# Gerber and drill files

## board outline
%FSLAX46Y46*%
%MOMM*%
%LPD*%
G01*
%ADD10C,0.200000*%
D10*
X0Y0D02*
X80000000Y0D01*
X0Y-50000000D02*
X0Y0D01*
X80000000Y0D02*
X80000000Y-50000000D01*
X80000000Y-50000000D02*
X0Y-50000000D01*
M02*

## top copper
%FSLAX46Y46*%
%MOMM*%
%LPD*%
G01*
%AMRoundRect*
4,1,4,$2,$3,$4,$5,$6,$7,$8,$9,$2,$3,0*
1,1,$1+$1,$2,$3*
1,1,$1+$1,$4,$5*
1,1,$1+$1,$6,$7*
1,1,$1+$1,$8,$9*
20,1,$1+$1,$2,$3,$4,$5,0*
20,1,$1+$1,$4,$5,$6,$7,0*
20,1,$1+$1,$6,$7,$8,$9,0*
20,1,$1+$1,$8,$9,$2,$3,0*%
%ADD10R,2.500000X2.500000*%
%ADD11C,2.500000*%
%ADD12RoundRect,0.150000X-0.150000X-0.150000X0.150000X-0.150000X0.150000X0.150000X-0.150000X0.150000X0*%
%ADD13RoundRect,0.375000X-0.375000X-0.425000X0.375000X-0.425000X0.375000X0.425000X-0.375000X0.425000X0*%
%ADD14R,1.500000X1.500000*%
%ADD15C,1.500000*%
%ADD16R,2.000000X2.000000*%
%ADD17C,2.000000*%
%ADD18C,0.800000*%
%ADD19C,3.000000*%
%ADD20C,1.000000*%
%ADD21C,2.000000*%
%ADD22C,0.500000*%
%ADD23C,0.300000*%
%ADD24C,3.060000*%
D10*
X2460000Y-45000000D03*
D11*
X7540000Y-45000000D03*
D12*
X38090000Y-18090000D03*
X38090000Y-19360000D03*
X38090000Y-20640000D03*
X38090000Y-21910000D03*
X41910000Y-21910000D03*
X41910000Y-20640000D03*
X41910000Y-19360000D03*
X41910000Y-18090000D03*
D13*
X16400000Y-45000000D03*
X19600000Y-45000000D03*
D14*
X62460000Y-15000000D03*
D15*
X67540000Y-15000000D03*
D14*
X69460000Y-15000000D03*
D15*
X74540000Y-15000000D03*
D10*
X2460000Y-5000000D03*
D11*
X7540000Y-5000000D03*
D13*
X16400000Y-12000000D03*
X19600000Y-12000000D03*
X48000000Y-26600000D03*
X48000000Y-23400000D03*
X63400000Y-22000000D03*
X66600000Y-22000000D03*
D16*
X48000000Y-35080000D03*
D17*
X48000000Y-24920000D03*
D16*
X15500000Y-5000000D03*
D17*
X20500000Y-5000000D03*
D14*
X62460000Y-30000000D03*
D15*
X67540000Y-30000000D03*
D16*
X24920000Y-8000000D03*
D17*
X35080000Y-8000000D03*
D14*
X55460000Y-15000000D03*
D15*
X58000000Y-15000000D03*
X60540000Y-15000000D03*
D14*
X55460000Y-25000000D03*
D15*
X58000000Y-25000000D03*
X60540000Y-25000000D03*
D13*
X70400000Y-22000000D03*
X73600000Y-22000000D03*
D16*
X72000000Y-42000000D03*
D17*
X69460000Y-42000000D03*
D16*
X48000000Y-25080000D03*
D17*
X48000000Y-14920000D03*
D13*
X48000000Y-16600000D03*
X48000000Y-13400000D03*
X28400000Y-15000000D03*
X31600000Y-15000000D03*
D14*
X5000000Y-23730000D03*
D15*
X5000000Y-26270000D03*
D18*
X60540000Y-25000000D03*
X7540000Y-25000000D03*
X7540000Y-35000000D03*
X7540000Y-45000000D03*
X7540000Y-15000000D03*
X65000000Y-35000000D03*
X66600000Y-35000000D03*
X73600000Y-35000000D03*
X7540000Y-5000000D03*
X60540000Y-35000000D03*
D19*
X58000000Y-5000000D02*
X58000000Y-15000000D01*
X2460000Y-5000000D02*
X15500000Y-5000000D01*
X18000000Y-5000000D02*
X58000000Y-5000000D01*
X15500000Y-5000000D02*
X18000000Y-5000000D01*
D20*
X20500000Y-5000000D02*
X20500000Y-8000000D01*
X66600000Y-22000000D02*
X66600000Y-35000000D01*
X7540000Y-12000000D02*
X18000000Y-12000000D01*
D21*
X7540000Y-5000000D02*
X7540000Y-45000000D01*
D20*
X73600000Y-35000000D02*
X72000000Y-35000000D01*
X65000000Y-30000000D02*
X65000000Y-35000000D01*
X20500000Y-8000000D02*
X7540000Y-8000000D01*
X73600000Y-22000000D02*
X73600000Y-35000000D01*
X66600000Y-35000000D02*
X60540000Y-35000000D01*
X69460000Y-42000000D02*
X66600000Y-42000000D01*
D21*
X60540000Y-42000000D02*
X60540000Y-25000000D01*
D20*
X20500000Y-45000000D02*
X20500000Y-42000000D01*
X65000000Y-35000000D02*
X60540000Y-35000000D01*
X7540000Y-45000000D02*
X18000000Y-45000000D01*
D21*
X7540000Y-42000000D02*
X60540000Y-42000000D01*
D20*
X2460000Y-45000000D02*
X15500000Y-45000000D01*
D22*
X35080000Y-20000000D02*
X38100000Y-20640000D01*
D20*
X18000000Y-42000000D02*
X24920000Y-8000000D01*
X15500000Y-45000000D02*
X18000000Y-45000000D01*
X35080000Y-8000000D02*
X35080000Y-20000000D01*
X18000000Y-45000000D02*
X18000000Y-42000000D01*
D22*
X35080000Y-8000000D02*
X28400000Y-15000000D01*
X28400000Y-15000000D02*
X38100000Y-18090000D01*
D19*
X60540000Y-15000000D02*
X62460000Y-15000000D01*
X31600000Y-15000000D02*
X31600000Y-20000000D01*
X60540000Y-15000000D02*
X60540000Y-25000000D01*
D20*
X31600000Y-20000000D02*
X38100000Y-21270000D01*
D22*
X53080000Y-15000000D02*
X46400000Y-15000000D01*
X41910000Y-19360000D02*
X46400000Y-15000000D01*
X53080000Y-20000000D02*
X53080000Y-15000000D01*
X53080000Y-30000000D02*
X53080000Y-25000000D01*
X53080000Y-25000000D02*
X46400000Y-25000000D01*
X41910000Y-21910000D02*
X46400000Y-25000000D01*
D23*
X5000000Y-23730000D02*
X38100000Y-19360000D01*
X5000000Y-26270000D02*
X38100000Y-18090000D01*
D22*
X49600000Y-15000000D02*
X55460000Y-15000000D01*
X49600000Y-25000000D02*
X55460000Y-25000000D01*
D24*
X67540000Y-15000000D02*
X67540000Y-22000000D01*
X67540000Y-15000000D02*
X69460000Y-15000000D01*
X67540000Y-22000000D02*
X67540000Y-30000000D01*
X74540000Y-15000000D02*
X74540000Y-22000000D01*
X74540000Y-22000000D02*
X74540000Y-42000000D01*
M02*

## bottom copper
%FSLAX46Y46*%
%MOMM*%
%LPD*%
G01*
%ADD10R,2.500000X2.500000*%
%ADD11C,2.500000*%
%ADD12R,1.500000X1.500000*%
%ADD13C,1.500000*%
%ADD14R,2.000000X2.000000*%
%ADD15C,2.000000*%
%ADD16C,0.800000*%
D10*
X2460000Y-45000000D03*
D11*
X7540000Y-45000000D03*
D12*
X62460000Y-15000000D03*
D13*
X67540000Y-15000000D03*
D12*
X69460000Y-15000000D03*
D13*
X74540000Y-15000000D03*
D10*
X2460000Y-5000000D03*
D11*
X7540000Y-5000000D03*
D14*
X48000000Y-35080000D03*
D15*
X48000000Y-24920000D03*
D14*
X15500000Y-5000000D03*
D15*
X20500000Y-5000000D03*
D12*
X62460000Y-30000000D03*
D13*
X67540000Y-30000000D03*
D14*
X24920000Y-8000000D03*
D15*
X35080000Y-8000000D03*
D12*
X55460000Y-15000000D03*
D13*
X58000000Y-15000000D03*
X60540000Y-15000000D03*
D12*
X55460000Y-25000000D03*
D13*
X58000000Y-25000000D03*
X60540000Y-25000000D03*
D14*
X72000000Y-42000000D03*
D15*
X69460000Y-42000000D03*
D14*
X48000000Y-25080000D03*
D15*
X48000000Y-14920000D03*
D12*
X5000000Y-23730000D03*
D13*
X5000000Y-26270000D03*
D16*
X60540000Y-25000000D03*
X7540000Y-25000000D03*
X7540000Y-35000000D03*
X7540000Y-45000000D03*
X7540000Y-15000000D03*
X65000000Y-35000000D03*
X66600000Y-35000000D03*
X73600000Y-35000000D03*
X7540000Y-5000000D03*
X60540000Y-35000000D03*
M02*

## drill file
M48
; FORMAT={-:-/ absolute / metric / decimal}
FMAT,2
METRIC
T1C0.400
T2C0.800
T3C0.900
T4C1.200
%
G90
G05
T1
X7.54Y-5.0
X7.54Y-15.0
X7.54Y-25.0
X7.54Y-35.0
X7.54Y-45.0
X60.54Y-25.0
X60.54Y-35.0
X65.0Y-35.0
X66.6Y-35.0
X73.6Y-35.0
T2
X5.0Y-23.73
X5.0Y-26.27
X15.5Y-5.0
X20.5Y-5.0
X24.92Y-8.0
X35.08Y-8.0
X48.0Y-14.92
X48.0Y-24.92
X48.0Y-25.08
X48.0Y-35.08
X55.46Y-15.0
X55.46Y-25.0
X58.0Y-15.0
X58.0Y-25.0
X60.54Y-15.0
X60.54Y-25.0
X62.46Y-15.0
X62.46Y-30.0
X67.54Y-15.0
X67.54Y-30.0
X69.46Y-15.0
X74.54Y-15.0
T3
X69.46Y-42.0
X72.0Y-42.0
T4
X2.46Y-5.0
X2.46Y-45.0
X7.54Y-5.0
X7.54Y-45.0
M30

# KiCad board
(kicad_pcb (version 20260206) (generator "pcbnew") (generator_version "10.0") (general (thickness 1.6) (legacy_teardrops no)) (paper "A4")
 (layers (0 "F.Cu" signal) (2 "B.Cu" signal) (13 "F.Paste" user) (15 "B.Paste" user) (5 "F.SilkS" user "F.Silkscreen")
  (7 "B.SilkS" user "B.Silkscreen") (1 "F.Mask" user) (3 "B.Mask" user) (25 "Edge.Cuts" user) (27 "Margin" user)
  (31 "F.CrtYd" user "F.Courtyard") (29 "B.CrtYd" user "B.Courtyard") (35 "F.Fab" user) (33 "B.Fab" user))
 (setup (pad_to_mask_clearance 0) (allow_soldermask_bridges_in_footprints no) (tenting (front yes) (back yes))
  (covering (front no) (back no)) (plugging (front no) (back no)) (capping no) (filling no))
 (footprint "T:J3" (layer "F.Cu") (at 5 45)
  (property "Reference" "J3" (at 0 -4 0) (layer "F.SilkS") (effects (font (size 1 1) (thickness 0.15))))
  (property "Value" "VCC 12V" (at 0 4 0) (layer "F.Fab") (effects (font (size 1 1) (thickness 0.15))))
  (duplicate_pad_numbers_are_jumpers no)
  (pad "1" thru_hole rect (at -2.54 0) (size 2.5 2.5) (drill 1.2) (layers "*.Cu" "*.Mask") (remove_unused_layers no) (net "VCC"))
  (pad "2" thru_hole circle (at 2.54 0) (size 2.5 2.5) (drill 1.2) (layers "*.Cu" "*.Mask") (remove_unused_layers no) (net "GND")))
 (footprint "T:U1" (layer "F.Cu") (at 40 20)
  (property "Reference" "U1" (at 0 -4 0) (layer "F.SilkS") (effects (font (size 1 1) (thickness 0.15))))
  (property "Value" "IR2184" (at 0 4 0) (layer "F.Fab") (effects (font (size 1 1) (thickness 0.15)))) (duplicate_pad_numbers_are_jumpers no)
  (pad "1" smd roundrect (at -1.91 -1.91) (size 0.6 0.6) (layers "F.Cu" "F.Mask" "F.Paste") (roundrect_rratio 0.25) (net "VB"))
  (pad "2" smd roundrect (at -1.91 -0.64) (size 0.6 0.6) (layers "F.Cu" "F.Mask" "F.Paste") (roundrect_rratio 0.25) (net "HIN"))
  (pad "3" smd roundrect (at -1.91 0.64) (size 0.6 0.6) (layers "F.Cu" "F.Mask" "F.Paste") (roundrect_rratio 0.25) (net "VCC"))
  (pad "4" smd roundrect (at -1.91 1.91) (size 0.6 0.6) (layers "F.Cu" "F.Mask" "F.Paste") (roundrect_rratio 0.25) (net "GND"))
  (pad "5" smd roundrect (at 1.91 1.91) (size 0.6 0.6) (layers "F.Cu" "F.Mask" "F.Paste") (roundrect_rratio 0.25) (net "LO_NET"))
  (pad "6" smd roundrect (at 1.91 0.64) (size 0.6 0.6) (layers "F.Cu" "F.Mask" "F.Paste") (roundrect_rratio 0.25) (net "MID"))
  (pad "7" smd roundrect (at 1.91 -0.64) (size 0.6 0.6) (layers "F.Cu" "F.Mask" "F.Paste") (roundrect_rratio 0.25) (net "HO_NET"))
  (pad "8" smd roundrect (at 1.91 -1.91) (size 0.6 0.6) (layers "F.Cu" "F.Mask" "F.Paste") (roundrect_rratio 0.25) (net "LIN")))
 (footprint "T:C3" (layer "F.Cu") (at 18 45)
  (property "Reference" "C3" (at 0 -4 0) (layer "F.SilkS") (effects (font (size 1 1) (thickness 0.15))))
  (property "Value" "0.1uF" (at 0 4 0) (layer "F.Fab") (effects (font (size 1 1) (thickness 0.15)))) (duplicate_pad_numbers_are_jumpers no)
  (pad "1" smd roundrect (at -1.6 0) (size 1.5 1.6) (layers "F.Cu" "F.Mask" "F.Paste") (roundrect_rratio 0.25) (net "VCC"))
  (pad "2" smd roundrect (at 1.6 0) (size 1.5 1.6) (layers "F.Cu" "F.Mask" "F.Paste") (roundrect_rratio 0.25) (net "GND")))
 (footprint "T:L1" (layer "F.Cu") (at 65 15)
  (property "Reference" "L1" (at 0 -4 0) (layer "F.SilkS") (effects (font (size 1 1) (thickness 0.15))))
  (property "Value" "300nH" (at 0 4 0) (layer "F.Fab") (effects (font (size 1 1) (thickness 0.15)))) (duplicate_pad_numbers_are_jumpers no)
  (pad "1" thru_hole rect (at -2.54 0) (size 1.5 1.5) (drill 0.8) (layers "*.Cu" "*.Mask") (remove_unused_layers no) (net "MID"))
  (pad "2" thru_hole circle (at 2.54 0) (size 1.5 1.5) (drill 0.8) (layers "*.Cu" "*.Mask") (remove_unused_layers no) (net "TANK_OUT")))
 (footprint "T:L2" (layer "F.Cu") (at 72 15)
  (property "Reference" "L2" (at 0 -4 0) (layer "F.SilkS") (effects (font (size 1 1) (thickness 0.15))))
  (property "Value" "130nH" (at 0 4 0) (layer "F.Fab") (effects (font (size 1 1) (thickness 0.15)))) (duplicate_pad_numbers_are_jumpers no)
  (pad "1" thru_hole rect (at -2.54 0) (size 1.5 1.5) (drill 0.8) (layers "*.Cu" "*.Mask") (remove_unused_layers no) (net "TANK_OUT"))
  (pad "2" thru_hole circle (at 2.54 0) (size 1.5 1.5) (drill 0.8) (layers "*.Cu" "*.Mask") (remove_unused_layers no) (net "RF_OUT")))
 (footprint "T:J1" (layer "F.Cu") (at 5 5)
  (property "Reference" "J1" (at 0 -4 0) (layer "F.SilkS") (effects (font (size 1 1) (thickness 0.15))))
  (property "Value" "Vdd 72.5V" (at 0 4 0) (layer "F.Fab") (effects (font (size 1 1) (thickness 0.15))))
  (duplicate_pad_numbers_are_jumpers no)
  (pad "1" thru_hole rect (at -2.54 0) (size 2.5 2.5) (drill 1.2) (layers "*.Cu" "*.Mask") (remove_unused_layers no) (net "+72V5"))
  (pad "2" thru_hole circle (at 2.54 0) (size 2.5 2.5) (drill 1.2) (layers "*.Cu" "*.Mask") (remove_unused_layers no) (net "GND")))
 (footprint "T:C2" (layer "F.Cu") (at 18 12)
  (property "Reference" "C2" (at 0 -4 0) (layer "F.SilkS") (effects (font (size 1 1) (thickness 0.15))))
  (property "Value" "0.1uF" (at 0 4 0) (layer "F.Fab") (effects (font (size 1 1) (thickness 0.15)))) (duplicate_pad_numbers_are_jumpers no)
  (pad "1" smd roundrect (at -1.6 0) (size 1.5 1.6) (layers "F.Cu" "F.Mask" "F.Paste") (roundrect_rratio 0.25) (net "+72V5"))
  (pad "2" smd roundrect (at 1.6 0) (size 1.5 1.6) (layers "F.Cu" "F.Mask" "F.Paste") (roundrect_rratio 0.25) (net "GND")))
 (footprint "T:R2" (layer "F.Cu") (at 48 25 90)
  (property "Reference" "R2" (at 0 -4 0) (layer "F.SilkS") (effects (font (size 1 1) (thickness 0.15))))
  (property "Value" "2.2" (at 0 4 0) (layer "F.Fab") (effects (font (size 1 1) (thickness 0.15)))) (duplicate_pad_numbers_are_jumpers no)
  (pad "1" smd roundrect (at -1.6 0) (size 1.5 1.6) (layers "F.Cu" "F.Mask" "F.Paste") (roundrect_rratio 0.25) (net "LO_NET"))
  (pad "2" smd roundrect (at 1.6 0) (size 1.5 1.6) (layers "F.Cu" "F.Mask" "F.Paste") (roundrect_rratio 0.25) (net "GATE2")))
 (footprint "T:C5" (layer "F.Cu") (at 65 22)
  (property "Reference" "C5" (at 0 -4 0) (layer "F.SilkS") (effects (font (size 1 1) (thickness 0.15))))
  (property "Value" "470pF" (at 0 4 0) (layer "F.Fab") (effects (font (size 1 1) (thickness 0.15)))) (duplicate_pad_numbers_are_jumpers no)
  (pad "1" smd roundrect (at -1.6 0) (size 1.5 1.6) (layers "F.Cu" "F.Mask" "F.Paste") (roundrect_rratio 0.25) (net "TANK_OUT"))
  (pad "2" smd roundrect (at 1.6 0) (size 1.5 1.6) (layers "F.Cu" "F.Mask" "F.Paste") (roundrect_rratio 0.25) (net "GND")))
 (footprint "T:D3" (layer "F.Cu") (at 48 30 90)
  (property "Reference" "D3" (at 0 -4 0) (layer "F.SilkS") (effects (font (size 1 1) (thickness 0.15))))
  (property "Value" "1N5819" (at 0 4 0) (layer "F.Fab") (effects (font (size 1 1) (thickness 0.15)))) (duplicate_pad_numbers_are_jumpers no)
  (pad "1" thru_hole rect (at -5.08 0) (size 2 2) (drill 0.8) (layers "*.Cu" "*.Mask") (remove_unused_layers no) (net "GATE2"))
  (pad "2" thru_hole circle (at 5.08 0) (size 2 2) (drill 0.8) (layers "*.Cu" "*.Mask") (remove_unused_layers no) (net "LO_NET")))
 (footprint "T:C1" (layer "F.Cu") (at 18 5)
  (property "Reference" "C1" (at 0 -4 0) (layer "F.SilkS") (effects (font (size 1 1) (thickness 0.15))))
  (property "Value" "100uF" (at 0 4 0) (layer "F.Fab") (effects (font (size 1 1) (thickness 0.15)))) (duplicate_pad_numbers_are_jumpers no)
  (pad "1" thru_hole rect (at -2.5 0) (size 2 2) (drill 0.8) (layers "*.Cu" "*.Mask") (remove_unused_layers no) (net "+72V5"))
  (pad "2" thru_hole circle (at 2.5 0) (size 2 2) (drill 0.8) (layers "*.Cu" "*.Mask") (remove_unused_layers no) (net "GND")))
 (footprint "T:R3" (layer "F.Cu") (at 65 30)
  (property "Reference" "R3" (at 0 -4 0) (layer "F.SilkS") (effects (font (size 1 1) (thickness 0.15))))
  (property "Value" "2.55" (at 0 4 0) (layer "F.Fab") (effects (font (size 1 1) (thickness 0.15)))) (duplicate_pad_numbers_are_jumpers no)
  (pad "1" thru_hole rect (at -2.54 0) (size 1.5 1.5) (drill 0.8) (layers "*.Cu" "*.Mask") (remove_unused_layers no) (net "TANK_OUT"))
  (pad "2" thru_hole circle (at 2.54 0) (size 1.5 1.5) (drill 0.8) (layers "*.Cu" "*.Mask") (remove_unused_layers no) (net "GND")))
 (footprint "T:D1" (layer "F.Cu") (at 30 8)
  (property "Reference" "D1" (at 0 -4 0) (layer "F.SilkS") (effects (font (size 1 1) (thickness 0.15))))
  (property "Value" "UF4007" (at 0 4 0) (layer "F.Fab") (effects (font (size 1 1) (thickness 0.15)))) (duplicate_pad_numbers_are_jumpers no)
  (pad "1" thru_hole rect (at -5.08 0) (size 2 2) (drill 0.8) (layers "*.Cu" "*.Mask") (remove_unused_layers no) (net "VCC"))
  (pad "2" thru_hole circle (at 5.08 0) (size 2 2) (drill 0.8) (layers "*.Cu" "*.Mask") (remove_unused_layers no) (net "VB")))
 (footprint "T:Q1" (layer "F.Cu") (at 58 15)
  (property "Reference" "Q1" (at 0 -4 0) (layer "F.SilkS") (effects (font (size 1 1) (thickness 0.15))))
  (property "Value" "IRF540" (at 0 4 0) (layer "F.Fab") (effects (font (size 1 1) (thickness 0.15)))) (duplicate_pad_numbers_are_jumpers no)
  (pad "1" thru_hole rect (at -2.54 0) (size 1.5 1.5) (drill 0.8) (layers "*.Cu" "*.Mask") (remove_unused_layers no) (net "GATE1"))
  (pad "2" thru_hole circle (at 0 0) (size 1.5 1.5) (drill 0.8) (layers "*.Cu" "*.Mask") (remove_unused_layers no) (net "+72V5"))
  (pad "3" thru_hole circle (at 2.54 0) (size 1.5 1.5) (drill 0.8) (layers "*.Cu" "*.Mask") (remove_unused_layers no) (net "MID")))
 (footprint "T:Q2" (layer "F.Cu") (at 58 25)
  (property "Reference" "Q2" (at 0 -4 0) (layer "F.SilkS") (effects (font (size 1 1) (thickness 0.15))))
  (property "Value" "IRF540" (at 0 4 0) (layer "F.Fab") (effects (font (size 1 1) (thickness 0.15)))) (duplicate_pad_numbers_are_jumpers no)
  (pad "1" thru_hole rect (at -2.54 0) (size 1.5 1.5) (drill 0.8) (layers "*.Cu" "*.Mask") (remove_unused_layers no) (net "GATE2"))
  (pad "2" thru_hole circle (at 0 0) (size 1.5 1.5) (drill 0.8) (layers "*.Cu" "*.Mask") (remove_unused_layers no) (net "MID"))
  (pad "3" thru_hole circle (at 2.54 0) (size 1.5 1.5) (drill 0.8) (layers "*.Cu" "*.Mask") (remove_unused_layers no) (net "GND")))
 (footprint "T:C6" (layer "F.Cu") (at 72 22)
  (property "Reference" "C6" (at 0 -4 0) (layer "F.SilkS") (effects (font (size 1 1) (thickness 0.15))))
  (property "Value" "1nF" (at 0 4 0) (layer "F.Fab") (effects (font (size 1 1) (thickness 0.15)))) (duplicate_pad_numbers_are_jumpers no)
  (pad "1" smd roundrect (at -1.6 0) (size 1.5 1.6) (layers "F.Cu" "F.Mask" "F.Paste") (roundrect_rratio 0.25) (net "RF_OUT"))
  (pad "2" smd roundrect (at 1.6 0) (size 1.5 1.6) (layers "F.Cu" "F.Mask" "F.Paste") (roundrect_rratio 0.25) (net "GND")))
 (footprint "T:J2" (layer "F.Cu") (at 72 42)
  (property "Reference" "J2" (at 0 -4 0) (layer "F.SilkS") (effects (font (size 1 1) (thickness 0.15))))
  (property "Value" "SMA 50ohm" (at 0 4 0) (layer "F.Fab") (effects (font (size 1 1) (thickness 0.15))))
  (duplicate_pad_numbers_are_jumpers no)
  (pad "1" thru_hole rect (at 0 0) (size 2 2) (drill 0.9) (layers "*.Cu" "*.Mask") (remove_unused_layers no) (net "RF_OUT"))
  (pad "2" thru_hole circle (at -2.54 0) (size 2 2) (drill 0.9) (layers "*.Cu" "*.Mask") (remove_unused_layers no) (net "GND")))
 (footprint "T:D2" (layer "F.Cu") (at 48 20 90)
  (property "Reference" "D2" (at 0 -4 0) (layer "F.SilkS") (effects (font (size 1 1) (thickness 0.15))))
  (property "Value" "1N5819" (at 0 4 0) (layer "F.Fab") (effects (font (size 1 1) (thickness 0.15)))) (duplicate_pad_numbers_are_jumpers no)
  (pad "1" thru_hole rect (at -5.08 0) (size 2 2) (drill 0.8) (layers "*.Cu" "*.Mask") (remove_unused_layers no) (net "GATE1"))
  (pad "2" thru_hole circle (at 5.08 0) (size 2 2) (drill 0.8) (layers "*.Cu" "*.Mask") (remove_unused_layers no) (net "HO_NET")))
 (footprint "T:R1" (layer "F.Cu") (at 48 15 90)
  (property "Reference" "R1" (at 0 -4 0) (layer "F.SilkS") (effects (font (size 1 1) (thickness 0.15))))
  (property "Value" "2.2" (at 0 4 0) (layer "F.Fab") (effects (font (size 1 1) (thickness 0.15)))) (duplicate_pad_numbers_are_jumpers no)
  (pad "1" smd roundrect (at -1.6 0) (size 1.5 1.6) (layers "F.Cu" "F.Mask" "F.Paste") (roundrect_rratio 0.25) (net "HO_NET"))
  (pad "2" smd roundrect (at 1.6 0) (size 1.5 1.6) (layers "F.Cu" "F.Mask" "F.Paste") (roundrect_rratio 0.25) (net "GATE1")))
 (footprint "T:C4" (layer "F.Cu") (at 30 15)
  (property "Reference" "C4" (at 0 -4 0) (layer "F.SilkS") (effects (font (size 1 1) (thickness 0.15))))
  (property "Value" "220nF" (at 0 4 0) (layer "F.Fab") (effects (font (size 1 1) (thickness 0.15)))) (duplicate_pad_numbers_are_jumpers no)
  (pad "1" smd roundrect (at -1.6 0) (size 1.5 1.6) (layers "F.Cu" "F.Mask" "F.Paste") (roundrect_rratio 0.25) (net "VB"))
  (pad "2" smd roundrect (at 1.6 0) (size 1.5 1.6) (layers "F.Cu" "F.Mask" "F.Paste") (roundrect_rratio 0.25) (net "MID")))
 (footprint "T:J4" (layer "F.Cu") (at 5 25)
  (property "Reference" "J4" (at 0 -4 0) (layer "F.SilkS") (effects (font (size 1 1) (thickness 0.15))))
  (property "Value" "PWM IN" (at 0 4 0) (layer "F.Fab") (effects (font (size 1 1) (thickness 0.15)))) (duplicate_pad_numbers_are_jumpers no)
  (pad "1" thru_hole rect (at 0 -1.27) (size 1.5 1.5) (drill 0.8) (layers "*.Cu" "*.Mask") (remove_unused_layers no) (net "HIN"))
  (pad "2" thru_hole circle (at 0 1.27) (size 1.5 1.5) (drill 0.8) (layers "*.Cu" "*.Mask") (remove_unused_layers no) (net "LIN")))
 (gr_line (start 0 0) (end 80 0) (stroke (width 0.2) (type default)) (layer "Edge.Cuts"))
 (gr_line (start 0 50) (end 0 0) (stroke (width 0.2) (type default)) (layer "Edge.Cuts"))
 (gr_line (start 80 0) (end 80 50) (stroke (width 0.2) (type default)) (layer "Edge.Cuts"))
 (gr_line (start 80 50) (end 0 50) (stroke (width 0.2) (type default)) (layer "Edge.Cuts"))
 (segment (start 58 5) (end 58 15) (width 3) (layer "F.Cu") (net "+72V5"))
 (segment (start 2.46 5) (end 15.5 5) (width 3) (layer "F.Cu") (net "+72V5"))
 (segment (start 18 5) (end 58 5) (width 3) (layer "F.Cu") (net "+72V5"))
 (segment (start 15.5 5) (end 18 5) (width 3) (layer "F.Cu") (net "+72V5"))
 (segment (start 20.5 5) (end 20.5 8) (width 1) (layer "F.Cu") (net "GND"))
 (segment (start 66.6 22) (end 66.6 35) (width 1) (layer "F.Cu") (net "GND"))
 (segment (start 7.54 12) (end 18 12) (width 1) (layer "F.Cu") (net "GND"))
 (segment (start 7.54 5) (end 7.54 45) (width 2) (layer "F.Cu") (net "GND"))
 (segment (start 73.6 35) (end 72 35) (width 1) (layer "F.Cu") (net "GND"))
 (segment (start 65 30) (end 65 35) (width 1) (layer "F.Cu") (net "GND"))
 (segment (start 20.5 8) (end 7.54 8) (width 1) (layer "F.Cu") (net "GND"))
 (segment (start 73.6 22) (end 73.6 35) (width 1) (layer "F.Cu") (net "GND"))
 (segment (start 66.6 35) (end 60.54 35) (width 1) (layer "F.Cu") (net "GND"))
 (segment (start 69.46 42) (end 66.6 42) (width 1) (layer "F.Cu") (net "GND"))
 (segment (start 60.54 42) (end 60.54 25) (width 2) (layer "F.Cu") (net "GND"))
 (segment (start 20.5 45) (end 20.5 42) (width 1) (layer "F.Cu") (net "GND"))
 (segment (start 65 35) (end 60.54 35) (width 1) (layer "F.Cu") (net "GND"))
 (segment (start 7.54 45) (end 18 45) (width 1) (layer "F.Cu") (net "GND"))
 (segment (start 7.54 42) (end 60.54 42) (width 2) (layer "F.Cu") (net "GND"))
 (via (at 60.54 25) (size 0.8) (drill 0.4) (layers "F.Cu" "B.Cu") (capping no) (covering (front no) (back no))
  (plugging (front no) (back no)) (filling no) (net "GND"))
 (via (at 7.54 25) (size 0.8) (drill 0.4) (layers "F.Cu" "B.Cu") (capping no) (covering (front no) (back no))
  (plugging (front no) (back no)) (filling no) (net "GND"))
 (via (at 7.54 35) (size 0.8) (drill 0.4) (layers "F.Cu" "B.Cu") (capping no) (covering (front no) (back no))
  (plugging (front no) (back no)) (filling no) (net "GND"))
 (via (at 7.54 45) (size 0.8) (drill 0.4) (layers "F.Cu" "B.Cu") (capping no) (covering (front no) (back no))
  (plugging (front no) (back no)) (filling no) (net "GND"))
 (via (at 7.54 15) (size 0.8) (drill 0.4) (layers "F.Cu" "B.Cu") (capping no) (covering (front no) (back no))
  (plugging (front no) (back no)) (filling no) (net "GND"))
 (via (at 65 35) (size 0.8) (drill 0.4) (layers "F.Cu" "B.Cu") (capping no) (covering (front no) (back no)) (plugging (front no) (back no))
  (filling no) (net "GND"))
 (via (at 66.6 35) (size 0.8) (drill 0.4) (layers "F.Cu" "B.Cu") (capping no) (covering (front no) (back no))
  (plugging (front no) (back no)) (filling no) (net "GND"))
 (via (at 73.6 35) (size 0.8) (drill 0.4) (layers "F.Cu" "B.Cu") (capping no) (covering (front no) (back no))
  (plugging (front no) (back no)) (filling no) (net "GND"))
 (via (at 7.54 5) (size 0.8) (drill 0.4) (layers "F.Cu" "B.Cu") (capping no) (covering (front no) (back no)) (plugging (front no) (back no))
  (filling no) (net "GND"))
 (via (at 60.54 35) (size 0.8) (drill 0.4) (layers "F.Cu" "B.Cu") (capping no) (covering (front no) (back no))
  (plugging (front no) (back no)) (filling no) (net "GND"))
 (segment (start 2.46 45) (end 15.5 45) (width 1) (layer "F.Cu") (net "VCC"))
 (segment (start 35.08 20) (end 38.1 20.64) (width 0.5) (layer "F.Cu") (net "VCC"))
 (segment (start 18 42) (end 24.92 8) (width 1) (layer "F.Cu") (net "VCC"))
 (segment (start 15.5 45) (end 18 45) (width 1) (layer "F.Cu") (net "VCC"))
 (segment (start 35.08 8) (end 35.08 20) (width 1) (layer "F.Cu") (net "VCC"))
 (segment (start 18 45) (end 18 42) (width 1) (layer "F.Cu") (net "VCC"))
 (segment (start 35.08 8) (end 28.4 15) (width 0.5) (layer "F.Cu") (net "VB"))
 (segment (start 28.4 15) (end 38.1 18.09) (width 0.5) (layer "F.Cu") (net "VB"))
 (segment (start 60.54 15) (end 62.46 15) (width 3) (layer "F.Cu") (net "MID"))
 (segment (start 31.6 15) (end 31.6 20) (width 3) (layer "F.Cu") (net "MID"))
 (segment (start 60.54 15) (end 60.54 25) (width 3) (layer "F.Cu") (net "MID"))
 (segment (start 31.6 20) (end 38.1 21.27) (width 1) (layer "F.Cu") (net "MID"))
 (segment (start 53.08 15) (end 46.4 15) (width 0.5) (layer "F.Cu") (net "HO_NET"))
 (segment (start 41.91 19.36) (end 46.4 15) (width 0.5) (layer "F.Cu") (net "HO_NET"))
 (segment (start 53.08 20) (end 53.08 15) (width 0.5) (layer "F.Cu") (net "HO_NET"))
 (segment (start 53.08 30) (end 53.08 25) (width 0.5) (layer "F.Cu") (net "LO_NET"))
 (segment (start 53.08 25) (end 46.4 25) (width 0.5) (layer "F.Cu") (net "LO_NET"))
 (segment (start 41.91 21.91) (end 46.4 25) (width 0.5) (layer "F.Cu") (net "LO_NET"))
 (segment (start 5 23.73) (end 38.1 19.36) (width 0.3) (layer "F.Cu") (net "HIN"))
 (segment (start 5 26.27) (end 38.1 18.09) (width 0.3) (layer "F.Cu") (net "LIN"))
 (segment (start 49.6 15) (end 55.46 15) (width 0.5) (layer "F.Cu") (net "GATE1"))
 (segment (start 49.6 25) (end 55.46 25) (width 0.5) (layer "F.Cu") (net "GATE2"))
 (segment (start 67.54 15) (end 67.54 22) (width 3.06) (layer "F.Cu") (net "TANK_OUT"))
 (segment (start 67.54 15) (end 69.46 15) (width 3.06) (layer "F.Cu") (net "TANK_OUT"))
 (segment (start 67.54 22) (end 67.54 30) (width 3.06) (layer "F.Cu") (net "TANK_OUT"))
 (segment (start 74.54 15) (end 74.54 22) (width 3.06) (layer "F.Cu") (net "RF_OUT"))
 (segment (start 74.54 22) (end 74.54 42) (width 3.06) (layer "F.Cu") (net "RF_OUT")))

